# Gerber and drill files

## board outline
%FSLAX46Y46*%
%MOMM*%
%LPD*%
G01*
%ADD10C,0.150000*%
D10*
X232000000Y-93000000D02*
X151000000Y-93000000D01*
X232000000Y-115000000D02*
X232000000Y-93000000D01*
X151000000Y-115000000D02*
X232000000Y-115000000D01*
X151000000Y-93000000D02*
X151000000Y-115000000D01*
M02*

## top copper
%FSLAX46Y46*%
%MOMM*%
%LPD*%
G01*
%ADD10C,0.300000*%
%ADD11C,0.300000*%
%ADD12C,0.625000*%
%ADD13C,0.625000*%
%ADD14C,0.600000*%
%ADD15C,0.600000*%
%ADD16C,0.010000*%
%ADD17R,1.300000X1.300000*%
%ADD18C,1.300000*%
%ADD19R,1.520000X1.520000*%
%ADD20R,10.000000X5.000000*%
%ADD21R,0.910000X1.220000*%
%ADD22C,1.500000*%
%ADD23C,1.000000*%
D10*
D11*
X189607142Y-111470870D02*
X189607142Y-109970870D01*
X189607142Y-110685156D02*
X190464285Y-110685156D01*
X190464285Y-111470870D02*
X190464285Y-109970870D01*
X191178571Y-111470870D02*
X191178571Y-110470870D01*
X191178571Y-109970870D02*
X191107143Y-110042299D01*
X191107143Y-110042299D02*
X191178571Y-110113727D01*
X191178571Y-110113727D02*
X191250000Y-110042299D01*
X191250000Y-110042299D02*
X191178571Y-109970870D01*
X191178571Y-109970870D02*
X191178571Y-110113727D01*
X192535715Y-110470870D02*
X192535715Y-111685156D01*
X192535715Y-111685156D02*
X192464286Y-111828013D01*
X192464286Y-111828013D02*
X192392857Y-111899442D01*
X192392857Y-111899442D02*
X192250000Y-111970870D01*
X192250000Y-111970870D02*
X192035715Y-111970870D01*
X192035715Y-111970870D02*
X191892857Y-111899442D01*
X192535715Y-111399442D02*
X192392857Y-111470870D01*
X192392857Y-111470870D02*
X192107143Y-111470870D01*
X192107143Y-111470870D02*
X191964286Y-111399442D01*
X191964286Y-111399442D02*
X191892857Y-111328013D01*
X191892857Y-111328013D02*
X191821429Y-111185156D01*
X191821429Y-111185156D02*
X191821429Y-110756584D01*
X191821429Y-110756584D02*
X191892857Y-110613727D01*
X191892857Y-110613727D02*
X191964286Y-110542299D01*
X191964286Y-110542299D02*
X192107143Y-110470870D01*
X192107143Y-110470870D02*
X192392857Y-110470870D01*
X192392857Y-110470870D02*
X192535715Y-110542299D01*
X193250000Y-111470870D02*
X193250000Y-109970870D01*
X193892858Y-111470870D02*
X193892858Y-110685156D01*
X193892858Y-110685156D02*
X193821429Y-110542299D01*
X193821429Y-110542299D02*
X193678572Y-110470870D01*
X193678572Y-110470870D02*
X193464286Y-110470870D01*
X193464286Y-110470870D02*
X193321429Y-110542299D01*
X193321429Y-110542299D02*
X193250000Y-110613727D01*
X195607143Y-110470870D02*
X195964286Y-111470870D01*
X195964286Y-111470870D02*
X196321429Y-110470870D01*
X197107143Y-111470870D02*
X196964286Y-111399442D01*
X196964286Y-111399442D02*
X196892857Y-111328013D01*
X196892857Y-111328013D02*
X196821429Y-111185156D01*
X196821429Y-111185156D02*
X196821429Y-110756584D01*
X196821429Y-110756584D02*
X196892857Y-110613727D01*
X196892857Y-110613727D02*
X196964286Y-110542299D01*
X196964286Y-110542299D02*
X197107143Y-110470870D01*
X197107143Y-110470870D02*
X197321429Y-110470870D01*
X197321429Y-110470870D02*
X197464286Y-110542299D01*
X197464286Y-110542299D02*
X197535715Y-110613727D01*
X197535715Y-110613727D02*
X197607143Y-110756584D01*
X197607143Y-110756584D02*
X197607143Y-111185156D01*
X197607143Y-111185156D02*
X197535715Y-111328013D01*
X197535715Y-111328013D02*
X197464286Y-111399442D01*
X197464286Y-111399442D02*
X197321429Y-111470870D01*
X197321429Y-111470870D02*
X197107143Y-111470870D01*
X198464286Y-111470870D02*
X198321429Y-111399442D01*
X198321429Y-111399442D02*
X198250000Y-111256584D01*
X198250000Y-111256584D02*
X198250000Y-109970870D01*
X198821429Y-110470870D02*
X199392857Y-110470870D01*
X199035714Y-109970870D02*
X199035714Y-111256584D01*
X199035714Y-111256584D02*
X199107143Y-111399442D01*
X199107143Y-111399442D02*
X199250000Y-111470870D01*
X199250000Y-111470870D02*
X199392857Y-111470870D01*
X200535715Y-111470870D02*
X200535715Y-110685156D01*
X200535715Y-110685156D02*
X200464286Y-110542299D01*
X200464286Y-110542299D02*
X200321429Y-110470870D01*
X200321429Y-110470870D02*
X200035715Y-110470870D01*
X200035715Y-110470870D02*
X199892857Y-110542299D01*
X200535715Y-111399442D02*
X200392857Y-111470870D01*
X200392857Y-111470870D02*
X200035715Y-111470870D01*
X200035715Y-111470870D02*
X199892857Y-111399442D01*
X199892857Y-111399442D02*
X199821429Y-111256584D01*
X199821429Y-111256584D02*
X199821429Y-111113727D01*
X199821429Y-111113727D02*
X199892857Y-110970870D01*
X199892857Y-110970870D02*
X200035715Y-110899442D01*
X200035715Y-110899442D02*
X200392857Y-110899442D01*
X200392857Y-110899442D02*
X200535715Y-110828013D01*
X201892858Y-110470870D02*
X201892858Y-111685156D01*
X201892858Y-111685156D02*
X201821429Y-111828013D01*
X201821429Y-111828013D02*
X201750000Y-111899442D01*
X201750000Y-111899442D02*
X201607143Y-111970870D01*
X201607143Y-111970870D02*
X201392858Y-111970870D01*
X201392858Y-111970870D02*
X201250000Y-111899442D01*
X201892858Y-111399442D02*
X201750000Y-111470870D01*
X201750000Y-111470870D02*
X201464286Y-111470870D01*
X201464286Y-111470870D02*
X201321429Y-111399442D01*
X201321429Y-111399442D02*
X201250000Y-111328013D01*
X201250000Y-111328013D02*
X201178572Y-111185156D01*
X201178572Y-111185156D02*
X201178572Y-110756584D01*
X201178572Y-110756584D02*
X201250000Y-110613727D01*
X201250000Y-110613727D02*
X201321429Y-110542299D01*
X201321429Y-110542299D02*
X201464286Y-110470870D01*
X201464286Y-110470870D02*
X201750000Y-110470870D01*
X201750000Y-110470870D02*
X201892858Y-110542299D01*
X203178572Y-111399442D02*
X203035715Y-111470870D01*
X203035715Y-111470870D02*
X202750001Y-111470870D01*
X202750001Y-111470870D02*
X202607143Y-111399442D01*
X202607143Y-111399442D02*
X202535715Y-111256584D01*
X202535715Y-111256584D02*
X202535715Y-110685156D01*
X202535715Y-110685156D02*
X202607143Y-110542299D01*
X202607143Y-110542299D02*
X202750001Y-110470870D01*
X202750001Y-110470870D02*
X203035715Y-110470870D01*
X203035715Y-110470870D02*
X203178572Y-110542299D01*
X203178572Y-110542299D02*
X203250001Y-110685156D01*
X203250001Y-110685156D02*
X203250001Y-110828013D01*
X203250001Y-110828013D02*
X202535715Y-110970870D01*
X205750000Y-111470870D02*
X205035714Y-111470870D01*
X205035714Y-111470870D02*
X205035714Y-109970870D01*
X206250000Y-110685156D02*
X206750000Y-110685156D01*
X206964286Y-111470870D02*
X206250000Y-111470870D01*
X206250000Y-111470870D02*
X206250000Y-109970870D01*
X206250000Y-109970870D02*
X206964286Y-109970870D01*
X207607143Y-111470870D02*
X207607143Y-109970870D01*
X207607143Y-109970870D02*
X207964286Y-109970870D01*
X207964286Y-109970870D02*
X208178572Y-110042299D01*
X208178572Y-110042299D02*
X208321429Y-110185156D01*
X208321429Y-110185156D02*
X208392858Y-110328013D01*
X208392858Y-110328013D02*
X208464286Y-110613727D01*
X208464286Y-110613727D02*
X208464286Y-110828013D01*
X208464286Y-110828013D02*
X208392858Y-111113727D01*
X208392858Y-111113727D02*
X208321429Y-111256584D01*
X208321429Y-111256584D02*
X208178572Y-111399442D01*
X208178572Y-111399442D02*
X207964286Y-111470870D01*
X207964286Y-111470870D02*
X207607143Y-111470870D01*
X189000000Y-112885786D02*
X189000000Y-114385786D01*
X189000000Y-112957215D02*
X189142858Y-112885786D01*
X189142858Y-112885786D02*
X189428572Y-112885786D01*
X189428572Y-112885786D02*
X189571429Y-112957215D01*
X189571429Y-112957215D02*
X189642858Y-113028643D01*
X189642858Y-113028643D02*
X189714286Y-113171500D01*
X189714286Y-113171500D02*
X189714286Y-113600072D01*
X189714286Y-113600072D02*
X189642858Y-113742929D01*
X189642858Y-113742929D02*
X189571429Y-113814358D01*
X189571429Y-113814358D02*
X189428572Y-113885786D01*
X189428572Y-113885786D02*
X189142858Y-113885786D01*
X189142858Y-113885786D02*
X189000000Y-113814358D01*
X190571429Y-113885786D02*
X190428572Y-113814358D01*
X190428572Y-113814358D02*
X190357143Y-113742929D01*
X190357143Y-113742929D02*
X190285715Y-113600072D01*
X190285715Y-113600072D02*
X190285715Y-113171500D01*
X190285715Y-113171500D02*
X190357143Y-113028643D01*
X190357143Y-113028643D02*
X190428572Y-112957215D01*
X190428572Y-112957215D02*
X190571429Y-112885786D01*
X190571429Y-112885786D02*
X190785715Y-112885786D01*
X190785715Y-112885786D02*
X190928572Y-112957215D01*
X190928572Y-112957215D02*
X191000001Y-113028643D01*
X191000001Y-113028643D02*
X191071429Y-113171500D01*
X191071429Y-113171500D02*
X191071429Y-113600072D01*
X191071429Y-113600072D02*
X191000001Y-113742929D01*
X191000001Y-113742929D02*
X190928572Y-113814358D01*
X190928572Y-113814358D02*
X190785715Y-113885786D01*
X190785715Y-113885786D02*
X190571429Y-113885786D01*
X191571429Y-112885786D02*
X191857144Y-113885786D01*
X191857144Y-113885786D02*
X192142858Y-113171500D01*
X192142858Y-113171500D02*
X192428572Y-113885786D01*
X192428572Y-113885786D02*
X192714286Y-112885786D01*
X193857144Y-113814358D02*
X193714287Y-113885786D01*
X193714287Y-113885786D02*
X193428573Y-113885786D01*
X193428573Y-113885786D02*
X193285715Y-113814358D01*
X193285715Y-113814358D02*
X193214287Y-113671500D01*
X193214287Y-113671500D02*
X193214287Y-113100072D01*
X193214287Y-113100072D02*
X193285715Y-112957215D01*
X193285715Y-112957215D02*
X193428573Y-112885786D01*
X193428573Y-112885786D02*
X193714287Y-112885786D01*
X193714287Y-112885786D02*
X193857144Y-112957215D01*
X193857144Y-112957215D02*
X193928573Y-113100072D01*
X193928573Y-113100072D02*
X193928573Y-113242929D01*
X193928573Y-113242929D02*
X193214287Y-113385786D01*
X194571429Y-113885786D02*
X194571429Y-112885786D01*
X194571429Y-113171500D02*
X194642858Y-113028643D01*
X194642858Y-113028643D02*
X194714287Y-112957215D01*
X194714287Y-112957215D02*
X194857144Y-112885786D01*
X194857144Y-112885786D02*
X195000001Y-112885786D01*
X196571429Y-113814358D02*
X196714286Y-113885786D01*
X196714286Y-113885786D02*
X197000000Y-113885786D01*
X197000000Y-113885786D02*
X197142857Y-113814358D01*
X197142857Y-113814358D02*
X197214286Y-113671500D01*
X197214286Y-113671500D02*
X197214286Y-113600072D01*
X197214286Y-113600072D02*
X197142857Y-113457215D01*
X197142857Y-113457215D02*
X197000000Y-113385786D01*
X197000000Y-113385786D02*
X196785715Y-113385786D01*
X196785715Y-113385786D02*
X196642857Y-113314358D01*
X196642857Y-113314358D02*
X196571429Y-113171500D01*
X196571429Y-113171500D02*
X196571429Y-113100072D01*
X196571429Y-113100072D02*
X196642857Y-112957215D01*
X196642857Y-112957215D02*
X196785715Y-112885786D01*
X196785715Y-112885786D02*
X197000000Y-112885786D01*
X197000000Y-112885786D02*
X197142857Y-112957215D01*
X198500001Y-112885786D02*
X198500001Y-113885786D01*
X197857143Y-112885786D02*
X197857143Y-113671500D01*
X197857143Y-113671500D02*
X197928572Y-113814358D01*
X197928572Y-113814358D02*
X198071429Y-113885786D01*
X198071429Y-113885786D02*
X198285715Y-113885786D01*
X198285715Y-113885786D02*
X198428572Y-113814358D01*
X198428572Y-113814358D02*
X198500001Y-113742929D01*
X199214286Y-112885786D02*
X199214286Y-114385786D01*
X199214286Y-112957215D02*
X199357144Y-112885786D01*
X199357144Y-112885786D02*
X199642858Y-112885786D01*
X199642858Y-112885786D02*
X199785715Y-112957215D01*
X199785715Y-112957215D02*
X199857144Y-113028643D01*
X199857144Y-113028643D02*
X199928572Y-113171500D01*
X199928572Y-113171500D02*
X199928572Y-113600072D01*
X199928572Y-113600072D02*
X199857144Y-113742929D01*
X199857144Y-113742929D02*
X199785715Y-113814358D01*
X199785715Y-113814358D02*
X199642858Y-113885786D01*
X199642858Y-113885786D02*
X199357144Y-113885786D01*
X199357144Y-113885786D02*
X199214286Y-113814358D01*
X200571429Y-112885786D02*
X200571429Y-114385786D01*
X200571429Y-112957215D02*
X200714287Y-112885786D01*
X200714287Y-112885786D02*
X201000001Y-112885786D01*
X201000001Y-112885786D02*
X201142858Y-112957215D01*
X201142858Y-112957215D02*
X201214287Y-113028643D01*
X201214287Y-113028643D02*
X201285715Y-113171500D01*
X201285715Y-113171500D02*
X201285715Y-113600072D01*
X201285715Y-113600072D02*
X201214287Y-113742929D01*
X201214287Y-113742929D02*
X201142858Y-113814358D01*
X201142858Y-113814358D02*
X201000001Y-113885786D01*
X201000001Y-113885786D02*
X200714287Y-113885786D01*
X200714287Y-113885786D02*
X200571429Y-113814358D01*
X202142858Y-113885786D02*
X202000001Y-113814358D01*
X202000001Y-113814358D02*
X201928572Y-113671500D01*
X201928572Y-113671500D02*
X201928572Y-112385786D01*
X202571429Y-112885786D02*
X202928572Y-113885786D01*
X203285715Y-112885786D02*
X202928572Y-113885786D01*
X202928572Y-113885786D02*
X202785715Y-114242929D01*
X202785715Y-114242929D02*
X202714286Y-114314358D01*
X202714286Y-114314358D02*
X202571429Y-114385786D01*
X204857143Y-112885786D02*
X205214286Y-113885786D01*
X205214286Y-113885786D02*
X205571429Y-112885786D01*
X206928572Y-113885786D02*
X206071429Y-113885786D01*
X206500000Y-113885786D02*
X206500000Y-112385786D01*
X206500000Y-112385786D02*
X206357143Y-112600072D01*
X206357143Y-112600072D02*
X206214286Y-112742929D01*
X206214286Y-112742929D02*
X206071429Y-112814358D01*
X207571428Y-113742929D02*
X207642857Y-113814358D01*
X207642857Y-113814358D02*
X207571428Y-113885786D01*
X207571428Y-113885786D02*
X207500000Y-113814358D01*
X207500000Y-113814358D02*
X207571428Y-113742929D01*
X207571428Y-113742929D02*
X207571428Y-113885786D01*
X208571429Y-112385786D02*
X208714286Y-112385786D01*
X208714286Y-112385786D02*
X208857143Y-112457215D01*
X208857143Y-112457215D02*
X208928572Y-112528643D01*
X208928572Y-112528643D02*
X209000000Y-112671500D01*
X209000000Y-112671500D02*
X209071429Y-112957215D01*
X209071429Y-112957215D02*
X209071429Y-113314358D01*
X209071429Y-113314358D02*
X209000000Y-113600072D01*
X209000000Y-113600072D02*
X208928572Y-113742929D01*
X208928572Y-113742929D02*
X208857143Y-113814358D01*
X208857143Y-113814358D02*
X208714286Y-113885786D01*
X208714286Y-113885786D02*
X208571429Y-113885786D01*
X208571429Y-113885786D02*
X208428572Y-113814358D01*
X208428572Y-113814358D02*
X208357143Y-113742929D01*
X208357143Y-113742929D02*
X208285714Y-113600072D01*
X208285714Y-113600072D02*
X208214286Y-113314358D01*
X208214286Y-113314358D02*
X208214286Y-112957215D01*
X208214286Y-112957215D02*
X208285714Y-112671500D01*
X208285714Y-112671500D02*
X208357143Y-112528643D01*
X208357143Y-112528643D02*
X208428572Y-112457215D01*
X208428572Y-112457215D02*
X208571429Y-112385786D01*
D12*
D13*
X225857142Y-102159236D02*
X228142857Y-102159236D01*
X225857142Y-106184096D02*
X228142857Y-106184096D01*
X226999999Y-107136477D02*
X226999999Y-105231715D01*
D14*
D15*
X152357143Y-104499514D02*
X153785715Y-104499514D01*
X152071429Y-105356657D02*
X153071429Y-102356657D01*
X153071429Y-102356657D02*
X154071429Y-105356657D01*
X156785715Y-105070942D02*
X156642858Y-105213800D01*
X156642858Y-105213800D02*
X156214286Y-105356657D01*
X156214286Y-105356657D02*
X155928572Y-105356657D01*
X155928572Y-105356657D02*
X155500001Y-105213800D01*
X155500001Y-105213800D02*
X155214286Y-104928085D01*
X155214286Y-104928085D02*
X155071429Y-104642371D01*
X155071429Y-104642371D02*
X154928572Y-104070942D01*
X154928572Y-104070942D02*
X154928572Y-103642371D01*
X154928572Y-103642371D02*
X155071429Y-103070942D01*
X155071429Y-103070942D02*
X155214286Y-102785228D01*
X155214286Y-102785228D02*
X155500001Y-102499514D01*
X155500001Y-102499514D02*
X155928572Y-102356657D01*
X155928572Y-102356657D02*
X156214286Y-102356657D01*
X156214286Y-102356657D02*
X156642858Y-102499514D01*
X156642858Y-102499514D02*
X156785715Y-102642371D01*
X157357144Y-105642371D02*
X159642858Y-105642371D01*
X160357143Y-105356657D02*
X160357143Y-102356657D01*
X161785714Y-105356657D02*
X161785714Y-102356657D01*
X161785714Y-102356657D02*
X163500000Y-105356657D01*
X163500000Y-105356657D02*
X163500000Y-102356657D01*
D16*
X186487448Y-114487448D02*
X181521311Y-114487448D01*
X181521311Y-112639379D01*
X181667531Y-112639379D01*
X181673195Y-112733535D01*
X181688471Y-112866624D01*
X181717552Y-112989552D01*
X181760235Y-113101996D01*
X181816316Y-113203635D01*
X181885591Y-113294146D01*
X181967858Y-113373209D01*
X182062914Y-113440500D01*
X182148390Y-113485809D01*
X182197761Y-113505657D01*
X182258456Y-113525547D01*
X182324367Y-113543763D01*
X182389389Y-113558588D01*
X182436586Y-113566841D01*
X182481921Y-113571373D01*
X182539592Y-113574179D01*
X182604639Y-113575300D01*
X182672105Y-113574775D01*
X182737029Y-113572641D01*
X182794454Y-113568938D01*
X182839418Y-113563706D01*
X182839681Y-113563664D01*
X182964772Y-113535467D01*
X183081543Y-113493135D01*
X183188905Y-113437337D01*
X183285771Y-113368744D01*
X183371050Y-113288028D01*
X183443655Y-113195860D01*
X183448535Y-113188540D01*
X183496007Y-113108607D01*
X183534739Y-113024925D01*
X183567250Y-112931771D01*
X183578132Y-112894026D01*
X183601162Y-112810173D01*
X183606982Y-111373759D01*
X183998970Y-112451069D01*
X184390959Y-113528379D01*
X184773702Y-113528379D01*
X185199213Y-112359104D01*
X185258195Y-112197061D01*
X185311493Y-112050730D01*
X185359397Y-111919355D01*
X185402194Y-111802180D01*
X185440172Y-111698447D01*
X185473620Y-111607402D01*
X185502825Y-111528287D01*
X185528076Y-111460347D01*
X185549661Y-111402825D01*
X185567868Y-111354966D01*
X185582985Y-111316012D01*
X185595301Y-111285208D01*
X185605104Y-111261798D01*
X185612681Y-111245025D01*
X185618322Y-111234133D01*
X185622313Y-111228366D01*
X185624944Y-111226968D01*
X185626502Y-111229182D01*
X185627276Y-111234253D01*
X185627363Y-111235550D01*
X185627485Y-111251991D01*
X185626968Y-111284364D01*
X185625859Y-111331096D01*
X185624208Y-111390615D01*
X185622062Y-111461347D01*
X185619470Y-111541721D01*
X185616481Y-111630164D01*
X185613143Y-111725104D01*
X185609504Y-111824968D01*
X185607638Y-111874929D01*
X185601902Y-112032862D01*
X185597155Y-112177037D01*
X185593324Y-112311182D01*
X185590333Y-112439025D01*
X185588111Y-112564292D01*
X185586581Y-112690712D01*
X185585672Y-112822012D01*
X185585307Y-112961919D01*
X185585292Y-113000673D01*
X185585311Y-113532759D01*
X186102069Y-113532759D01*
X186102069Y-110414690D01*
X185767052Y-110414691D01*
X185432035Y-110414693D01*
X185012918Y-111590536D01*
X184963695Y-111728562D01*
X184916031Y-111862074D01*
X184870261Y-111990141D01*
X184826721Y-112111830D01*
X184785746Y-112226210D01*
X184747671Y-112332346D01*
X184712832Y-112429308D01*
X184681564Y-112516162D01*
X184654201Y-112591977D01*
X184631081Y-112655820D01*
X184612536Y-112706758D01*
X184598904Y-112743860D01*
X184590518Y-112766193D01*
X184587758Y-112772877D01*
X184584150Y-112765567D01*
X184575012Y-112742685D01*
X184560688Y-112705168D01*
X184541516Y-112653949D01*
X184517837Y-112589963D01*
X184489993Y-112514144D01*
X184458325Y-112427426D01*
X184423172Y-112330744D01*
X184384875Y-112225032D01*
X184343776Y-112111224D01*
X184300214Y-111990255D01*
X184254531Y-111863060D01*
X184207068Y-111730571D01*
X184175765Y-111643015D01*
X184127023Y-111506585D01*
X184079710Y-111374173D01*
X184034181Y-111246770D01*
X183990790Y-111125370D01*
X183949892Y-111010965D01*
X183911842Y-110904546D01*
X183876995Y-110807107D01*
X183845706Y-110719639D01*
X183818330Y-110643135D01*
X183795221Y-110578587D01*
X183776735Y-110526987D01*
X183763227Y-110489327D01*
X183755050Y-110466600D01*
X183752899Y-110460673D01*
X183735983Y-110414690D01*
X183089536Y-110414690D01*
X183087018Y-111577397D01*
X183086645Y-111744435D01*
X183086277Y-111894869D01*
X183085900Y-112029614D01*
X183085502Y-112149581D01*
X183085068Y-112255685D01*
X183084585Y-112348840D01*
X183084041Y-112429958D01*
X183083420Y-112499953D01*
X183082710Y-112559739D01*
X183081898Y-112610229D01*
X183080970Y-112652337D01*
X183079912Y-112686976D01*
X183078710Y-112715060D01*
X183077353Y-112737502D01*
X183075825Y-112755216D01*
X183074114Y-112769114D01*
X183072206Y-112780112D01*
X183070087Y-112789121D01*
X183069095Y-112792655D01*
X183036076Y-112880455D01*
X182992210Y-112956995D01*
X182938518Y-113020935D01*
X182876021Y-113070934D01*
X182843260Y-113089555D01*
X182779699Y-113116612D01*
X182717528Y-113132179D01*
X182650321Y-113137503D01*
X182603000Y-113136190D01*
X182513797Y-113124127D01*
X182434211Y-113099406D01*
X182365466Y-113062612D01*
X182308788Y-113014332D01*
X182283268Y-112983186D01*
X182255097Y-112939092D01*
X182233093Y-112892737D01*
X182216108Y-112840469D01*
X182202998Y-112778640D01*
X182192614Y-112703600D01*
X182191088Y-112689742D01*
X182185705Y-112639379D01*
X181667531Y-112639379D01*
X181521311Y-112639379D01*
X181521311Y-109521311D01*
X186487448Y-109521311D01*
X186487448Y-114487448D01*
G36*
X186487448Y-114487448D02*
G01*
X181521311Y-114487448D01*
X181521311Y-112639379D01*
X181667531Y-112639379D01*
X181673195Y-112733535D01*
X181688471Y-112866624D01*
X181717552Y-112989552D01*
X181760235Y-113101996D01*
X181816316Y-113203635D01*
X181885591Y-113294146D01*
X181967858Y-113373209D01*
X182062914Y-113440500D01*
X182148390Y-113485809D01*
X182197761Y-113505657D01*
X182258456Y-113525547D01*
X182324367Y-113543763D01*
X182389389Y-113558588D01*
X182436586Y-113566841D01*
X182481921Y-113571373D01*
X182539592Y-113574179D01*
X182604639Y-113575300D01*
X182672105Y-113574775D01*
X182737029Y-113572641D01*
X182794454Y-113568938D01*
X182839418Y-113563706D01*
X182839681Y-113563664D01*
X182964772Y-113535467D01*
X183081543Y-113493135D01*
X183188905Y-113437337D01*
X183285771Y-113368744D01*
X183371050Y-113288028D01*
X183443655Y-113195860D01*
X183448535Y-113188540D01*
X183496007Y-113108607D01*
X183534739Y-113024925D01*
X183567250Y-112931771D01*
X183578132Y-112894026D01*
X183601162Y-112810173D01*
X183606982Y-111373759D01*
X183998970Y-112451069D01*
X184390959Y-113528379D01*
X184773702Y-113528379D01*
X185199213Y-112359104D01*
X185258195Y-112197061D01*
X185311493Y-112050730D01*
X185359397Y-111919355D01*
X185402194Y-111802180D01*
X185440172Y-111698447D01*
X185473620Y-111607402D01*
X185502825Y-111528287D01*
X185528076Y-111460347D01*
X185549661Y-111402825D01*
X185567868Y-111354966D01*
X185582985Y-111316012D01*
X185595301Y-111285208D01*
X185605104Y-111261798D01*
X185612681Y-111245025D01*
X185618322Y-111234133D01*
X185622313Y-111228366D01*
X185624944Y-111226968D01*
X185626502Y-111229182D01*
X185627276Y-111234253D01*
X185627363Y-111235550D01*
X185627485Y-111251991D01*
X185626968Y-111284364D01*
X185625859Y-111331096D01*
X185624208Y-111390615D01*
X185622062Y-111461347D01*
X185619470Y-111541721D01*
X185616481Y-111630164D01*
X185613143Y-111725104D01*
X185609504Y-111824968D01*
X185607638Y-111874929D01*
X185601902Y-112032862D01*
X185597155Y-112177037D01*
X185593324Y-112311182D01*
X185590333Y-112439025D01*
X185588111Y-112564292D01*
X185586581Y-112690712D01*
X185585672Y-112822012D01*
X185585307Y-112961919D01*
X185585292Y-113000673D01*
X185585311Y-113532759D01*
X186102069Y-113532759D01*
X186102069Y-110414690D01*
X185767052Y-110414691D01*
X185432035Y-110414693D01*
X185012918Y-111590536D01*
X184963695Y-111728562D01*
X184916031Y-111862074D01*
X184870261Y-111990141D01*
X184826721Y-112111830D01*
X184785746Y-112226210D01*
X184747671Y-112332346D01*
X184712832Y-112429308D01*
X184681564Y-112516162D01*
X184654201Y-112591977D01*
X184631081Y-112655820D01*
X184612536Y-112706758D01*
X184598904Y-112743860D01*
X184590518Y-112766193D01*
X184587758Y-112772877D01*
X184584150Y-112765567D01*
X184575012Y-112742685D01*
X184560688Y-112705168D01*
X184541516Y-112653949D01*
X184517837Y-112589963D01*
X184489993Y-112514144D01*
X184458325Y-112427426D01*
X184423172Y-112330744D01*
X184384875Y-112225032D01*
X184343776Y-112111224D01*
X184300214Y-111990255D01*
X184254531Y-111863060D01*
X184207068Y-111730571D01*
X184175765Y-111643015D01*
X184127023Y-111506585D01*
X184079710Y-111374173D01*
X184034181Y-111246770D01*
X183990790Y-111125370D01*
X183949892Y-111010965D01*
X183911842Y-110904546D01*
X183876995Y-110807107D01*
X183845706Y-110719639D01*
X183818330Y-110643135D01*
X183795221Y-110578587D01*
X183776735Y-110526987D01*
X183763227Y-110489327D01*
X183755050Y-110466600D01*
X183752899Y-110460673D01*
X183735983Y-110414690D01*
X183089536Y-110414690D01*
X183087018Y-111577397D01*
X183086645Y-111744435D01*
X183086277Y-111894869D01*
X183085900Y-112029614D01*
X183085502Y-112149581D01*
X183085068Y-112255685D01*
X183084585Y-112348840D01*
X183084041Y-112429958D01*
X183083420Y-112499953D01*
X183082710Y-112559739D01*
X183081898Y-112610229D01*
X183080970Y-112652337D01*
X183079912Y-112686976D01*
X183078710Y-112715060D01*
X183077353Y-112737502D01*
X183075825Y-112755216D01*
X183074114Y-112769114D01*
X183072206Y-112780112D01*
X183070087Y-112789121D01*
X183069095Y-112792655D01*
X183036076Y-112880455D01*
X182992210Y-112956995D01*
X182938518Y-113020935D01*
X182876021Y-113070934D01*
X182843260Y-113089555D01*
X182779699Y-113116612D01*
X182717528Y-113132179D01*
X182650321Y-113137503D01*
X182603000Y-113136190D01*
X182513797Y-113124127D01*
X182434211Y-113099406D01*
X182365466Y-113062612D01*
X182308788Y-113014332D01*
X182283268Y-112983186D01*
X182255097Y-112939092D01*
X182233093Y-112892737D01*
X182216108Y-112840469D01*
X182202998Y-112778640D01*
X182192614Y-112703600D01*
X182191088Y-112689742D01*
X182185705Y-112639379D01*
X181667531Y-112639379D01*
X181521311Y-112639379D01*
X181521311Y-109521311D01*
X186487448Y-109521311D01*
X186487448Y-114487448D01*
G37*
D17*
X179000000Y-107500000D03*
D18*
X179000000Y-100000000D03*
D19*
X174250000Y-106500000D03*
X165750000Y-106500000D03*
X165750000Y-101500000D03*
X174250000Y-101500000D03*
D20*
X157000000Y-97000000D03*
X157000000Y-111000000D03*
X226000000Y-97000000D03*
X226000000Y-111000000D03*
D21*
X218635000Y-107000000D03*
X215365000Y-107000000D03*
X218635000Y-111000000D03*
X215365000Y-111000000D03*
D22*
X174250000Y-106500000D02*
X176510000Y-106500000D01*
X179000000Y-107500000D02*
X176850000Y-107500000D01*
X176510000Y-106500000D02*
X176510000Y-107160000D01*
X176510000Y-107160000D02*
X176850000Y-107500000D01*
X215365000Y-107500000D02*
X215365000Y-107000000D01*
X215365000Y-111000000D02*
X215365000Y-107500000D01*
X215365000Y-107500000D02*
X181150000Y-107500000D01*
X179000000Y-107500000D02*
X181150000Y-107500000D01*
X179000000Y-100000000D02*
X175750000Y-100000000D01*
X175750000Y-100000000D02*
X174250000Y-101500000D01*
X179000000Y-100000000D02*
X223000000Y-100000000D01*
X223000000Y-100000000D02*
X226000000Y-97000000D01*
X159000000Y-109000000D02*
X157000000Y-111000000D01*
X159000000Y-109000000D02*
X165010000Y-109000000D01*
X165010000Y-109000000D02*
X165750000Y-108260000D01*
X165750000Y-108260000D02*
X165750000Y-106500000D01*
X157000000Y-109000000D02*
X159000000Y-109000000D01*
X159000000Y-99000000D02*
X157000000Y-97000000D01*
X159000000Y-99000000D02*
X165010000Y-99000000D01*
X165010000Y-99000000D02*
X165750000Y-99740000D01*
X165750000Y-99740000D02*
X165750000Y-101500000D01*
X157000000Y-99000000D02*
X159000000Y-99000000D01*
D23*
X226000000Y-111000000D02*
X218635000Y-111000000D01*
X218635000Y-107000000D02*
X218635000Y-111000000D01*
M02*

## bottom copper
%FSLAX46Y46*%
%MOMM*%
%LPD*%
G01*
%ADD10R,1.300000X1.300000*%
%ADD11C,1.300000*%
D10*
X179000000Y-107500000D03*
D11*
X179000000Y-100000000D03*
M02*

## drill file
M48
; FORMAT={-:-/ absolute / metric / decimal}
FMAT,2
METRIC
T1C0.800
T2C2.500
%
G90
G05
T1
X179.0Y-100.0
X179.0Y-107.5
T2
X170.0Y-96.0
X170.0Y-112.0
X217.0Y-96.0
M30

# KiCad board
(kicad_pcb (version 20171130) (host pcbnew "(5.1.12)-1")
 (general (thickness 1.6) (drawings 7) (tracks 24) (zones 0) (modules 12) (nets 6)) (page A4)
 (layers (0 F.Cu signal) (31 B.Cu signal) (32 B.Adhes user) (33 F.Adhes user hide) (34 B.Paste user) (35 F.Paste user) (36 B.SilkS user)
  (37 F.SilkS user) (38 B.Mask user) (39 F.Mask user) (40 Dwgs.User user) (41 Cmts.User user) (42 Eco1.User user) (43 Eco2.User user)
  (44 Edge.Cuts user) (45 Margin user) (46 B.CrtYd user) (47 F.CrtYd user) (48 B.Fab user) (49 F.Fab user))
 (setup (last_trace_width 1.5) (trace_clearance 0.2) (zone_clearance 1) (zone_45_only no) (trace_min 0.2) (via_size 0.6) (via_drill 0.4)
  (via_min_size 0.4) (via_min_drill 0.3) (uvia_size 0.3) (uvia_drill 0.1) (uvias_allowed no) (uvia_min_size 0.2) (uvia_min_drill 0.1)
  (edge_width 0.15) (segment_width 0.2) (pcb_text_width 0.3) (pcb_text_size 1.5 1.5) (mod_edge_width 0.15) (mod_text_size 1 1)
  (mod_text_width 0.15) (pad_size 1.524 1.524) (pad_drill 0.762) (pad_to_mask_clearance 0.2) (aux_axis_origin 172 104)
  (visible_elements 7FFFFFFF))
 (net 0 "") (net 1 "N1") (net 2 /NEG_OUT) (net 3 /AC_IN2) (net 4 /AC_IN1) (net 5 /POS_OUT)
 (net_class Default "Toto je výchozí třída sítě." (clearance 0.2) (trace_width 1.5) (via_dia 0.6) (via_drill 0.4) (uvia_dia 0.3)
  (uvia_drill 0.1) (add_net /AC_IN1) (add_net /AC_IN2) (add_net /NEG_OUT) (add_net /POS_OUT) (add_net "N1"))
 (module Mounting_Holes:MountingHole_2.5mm (layer F.Cu) (at 217 96)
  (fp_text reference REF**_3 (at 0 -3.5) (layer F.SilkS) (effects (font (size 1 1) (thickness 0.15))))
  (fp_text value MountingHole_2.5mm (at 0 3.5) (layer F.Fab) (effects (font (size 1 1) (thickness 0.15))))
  (pad 1 np_thru_hole circle (at 0 0) (size 2.5 2.5) (drill 2.5) (layers *.Cu *.Mask F.SilkS)))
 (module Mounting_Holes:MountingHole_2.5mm (layer F.Cu) (at 170 96)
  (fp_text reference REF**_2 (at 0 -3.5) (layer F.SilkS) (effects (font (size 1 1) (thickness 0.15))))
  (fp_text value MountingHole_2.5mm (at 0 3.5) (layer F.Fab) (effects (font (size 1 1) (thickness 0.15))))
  (pad 1 np_thru_hole circle (at 0 0) (size 2.5 2.5) (drill 2.5) (layers *.Cu *.Mask F.SilkS)))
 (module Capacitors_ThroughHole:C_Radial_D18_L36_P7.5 (layer F.Cu) (at 179 107.5 90)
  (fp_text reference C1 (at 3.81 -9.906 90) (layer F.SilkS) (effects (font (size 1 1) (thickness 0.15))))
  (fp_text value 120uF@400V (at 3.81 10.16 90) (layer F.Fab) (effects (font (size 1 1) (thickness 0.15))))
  (pad 1 thru_hole rect (at 0 0 90) (size 1.3 1.3) (drill 0.8) (layers *.Cu *.Mask F.SilkS) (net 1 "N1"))
  (pad 2 thru_hole circle (at 7.5 0 90) (size 1.3 1.3) (drill 0.8) (layers *.Cu *.Mask F.SilkS) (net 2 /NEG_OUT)))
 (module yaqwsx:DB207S (layer F.Cu) (at 170 104 270)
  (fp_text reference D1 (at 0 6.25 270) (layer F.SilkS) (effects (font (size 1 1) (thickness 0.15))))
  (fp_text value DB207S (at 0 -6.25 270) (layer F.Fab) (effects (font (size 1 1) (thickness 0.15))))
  (pad 3 smd rect (at 2.5 -4.25 270) (size 1.52 1.52) (layers F.Cu F.Paste F.Mask) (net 1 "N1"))
  (pad 4 smd rect (at 2.5 4.25 270) (size 1.52 1.52) (layers F.Cu F.Paste F.Mask) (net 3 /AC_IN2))
  (pad 2 smd rect (at -2.5 4.25 270) (size 1.52 1.52) (layers F.Cu F.Paste F.Mask) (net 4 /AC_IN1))
  (pad 1 smd rect (at -2.5 -4.25 270) (size 1.52 1.52) (layers F.Cu F.Paste F.Mask) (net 2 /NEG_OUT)))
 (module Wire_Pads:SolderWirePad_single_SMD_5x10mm (layer F.Cu) (at 157 97 90)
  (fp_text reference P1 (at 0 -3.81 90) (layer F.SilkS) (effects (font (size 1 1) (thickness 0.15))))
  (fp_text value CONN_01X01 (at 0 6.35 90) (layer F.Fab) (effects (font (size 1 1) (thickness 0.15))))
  (pad 1 smd rect (at 0 0 90) (size 5 10) (layers F.Cu F.Paste F.Mask) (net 4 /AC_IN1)))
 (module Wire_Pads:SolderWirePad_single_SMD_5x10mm (layer F.Cu) (at 157 111 90)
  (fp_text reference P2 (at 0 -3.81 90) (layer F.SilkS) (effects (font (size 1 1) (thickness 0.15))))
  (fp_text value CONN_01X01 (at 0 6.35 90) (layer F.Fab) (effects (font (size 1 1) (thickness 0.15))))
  (pad 1 smd rect (at 0 0 90) (size 5 10) (layers F.Cu F.Paste F.Mask) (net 3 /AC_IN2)))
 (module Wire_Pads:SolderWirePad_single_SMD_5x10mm (layer F.Cu) (at 226 97 90)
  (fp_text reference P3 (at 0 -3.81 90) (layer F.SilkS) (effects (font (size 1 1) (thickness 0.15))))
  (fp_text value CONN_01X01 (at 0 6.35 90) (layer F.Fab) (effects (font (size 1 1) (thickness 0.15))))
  (pad 1 smd rect (at 0 0 90) (size 5 10) (layers F.Cu F.Paste F.Mask) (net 2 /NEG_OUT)))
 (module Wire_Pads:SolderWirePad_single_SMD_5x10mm (layer F.Cu) (at 226 111 90)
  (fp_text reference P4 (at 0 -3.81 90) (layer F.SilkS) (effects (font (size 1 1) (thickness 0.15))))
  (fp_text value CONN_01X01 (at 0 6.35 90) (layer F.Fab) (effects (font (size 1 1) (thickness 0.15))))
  (pad 1 smd rect (at 0 0 90) (size 5 10) (layers F.Cu F.Paste F.Mask) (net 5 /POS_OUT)))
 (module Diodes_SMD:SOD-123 (layer F.Cu) (at 217 107 180)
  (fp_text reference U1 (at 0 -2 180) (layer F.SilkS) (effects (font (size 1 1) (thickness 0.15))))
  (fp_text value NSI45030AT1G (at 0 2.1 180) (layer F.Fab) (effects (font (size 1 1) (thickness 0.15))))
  (pad 1 smd rect (at -1.635 0 180) (size 0.91 1.22) (layers F.Cu F.Paste F.Mask) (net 5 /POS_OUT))
  (pad 2 smd rect (at 1.635 0 180) (size 0.91 1.22) (layers F.Cu F.Paste F.Mask) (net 1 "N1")))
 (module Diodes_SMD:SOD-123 (layer F.Cu) (at 217 111 180)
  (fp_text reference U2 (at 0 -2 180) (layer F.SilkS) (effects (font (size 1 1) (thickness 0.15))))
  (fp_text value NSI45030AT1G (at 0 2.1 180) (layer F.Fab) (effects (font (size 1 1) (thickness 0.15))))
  (pad 1 smd rect (at -1.635 0 180) (size 0.91 1.22) (layers F.Cu F.Paste F.Mask) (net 5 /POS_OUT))
  (pad 2 smd rect (at 1.635 0 180) (size 0.91 1.22) (layers F.Cu F.Paste F.Mask) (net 1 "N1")))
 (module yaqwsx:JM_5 (layer F.Cu) (at 184 112)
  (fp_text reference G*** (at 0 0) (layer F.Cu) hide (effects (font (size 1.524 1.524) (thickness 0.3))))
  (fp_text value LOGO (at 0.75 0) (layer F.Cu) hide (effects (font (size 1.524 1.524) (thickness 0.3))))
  (fp_poly
   (pts (xy 2.487448 2.487448) (xy -2.478689 2.487448) (xy -2.478689 0.639379) (xy -2.332469 0.639379) (xy -2.326805 0.733535)
    (xy -2.311529 0.866624) (xy -2.282448 0.989552) (xy -2.239765 1.101996) (xy -2.183684 1.203635) (xy -2.114409 1.294146)
    (xy -2.032142 1.373209) (xy -1.937086 1.4405) (xy -1.85161 1.485809) (xy -1.802239 1.505657) (xy -1.741544 1.525547)
    (xy -1.675633 1.543763) (xy -1.610611 1.558588) (xy -1.563414 1.566841) (xy -1.518079 1.571373) (xy -1.460408 1.574179)
    (xy -1.395361 1.5753) (xy -1.327895 1.574775) (xy -1.262971 1.572641) (xy -1.205546 1.568938) (xy -1.160582 1.563706)
    (xy -1.160319 1.563664) (xy -1.035228 1.535467) (xy -0.918457 1.493135) (xy -0.811095 1.437337) (xy -0.714229 1.368744)
    (xy -0.62895 1.288028) (xy -0.556345 1.19586) (xy -0.551465 1.18854) (xy -0.503993 1.108607) (xy -0.465261 1.024925)
    (xy -0.43275 0.931771) (xy -0.421868 0.894026) (xy -0.398838 0.810173) (xy -0.393018 -0.626241) (xy -0.00103 0.451069)
    (xy 0.390959 1.528379) (xy 0.773702 1.528379) (xy 1.199213 0.359104) (xy 1.258195 0.197061) (xy 1.311493 0.05073)
    (xy 1.359397 -0.080645) (xy 1.402194 -0.19782) (xy 1.440172 -0.301553) (xy 1.47362 -0.392598) (xy 1.502825 -0.471713)
    (xy 1.528076 -0.539653) (xy 1.549661 -0.597175) (xy 1.567868 -0.645034) (xy 1.582985 -0.683988) (xy 1.595301 -0.714792)
    (xy 1.605104 -0.738202) (xy 1.612681 -0.754975) (xy 1.618322 -0.765867) (xy 1.622313 -0.771634) (xy 1.624944 -0.773032)
    (xy 1.626502 -0.770818) (xy 1.627276 -0.765747) (xy 1.627363 -0.76445) (xy 1.627485 -0.748009) (xy 1.626968 -0.715636)
    (xy 1.625859 -0.668904) (xy 1.624208 -0.609385) (xy 1.622062 -0.538653) (xy 1.61947 -0.458279) (xy 1.616481 -0.369836)
    (xy 1.613143 -0.274896) (xy 1.609504 -0.175032) (xy 1.607638 -0.125071) (xy 1.601902 0.032862) (xy 1.597155 0.177037)
    (xy 1.593324 0.311182) (xy 1.590333 0.439025) (xy 1.588111 0.564292) (xy 1.586581 0.690712) (xy 1.585672 0.822012)
    (xy 1.585307 0.961919) (xy 1.585292 1.000673) (xy 1.585311 1.532759) (xy 2.102069 1.532759) (xy 2.102069 -1.58531)
    (xy 1.767052 -1.585309) (xy 1.432035 -1.585307) (xy 1.012918 -0.409464) (xy 0.963695 -0.271438) (xy 0.916031 -0.137926)
    (xy 0.870261 -0.009859) (xy 0.826721 0.11183) (xy 0.785746 0.22621) (xy 0.747671 0.332346) (xy 0.712832 0.429308) (xy 0.681564 0.516162)
    (xy 0.654201 0.591977) (xy 0.631081 0.65582) (xy 0.612536 0.706758) (xy 0.598904 0.74386) (xy 0.590518 0.766193) (xy 0.587758 0.772877)
    (xy 0.58415 0.765567) (xy 0.575012 0.742685) (xy 0.560688 0.705168) (xy 0.541516 0.653949) (xy 0.517837 0.589963) (xy 0.489993 0.514144)
    (xy 0.458325 0.427426) (xy 0.423172 0.330744) (xy 0.384875 0.225032) (xy 0.343776 0.111224) (xy 0.300214 -0.009745)
    (xy 0.254531 -0.13694) (xy 0.207068 -0.269429) (xy 0.175765 -0.356985) (xy 0.127023 -0.493415) (xy 0.07971 -0.625827)
    (xy 0.034181 -0.75323) (xy -0.00921 -0.87463) (xy -0.050108 -0.989035) (xy -0.088158 -1.095454) (xy -0.123005 -1.192893)
    (xy -0.154294 -1.280361) (xy -0.18167 -1.356865) (xy -0.204779 -1.421413) (xy -0.223265 -1.473013) (xy -0.236773 -1.510673)
    (xy -0.24495 -1.5334) (xy -0.247101 -1.539327) (xy -0.264017 -1.58531) (xy -0.910464 -1.58531) (xy -0.912982 -0.422603)
    (xy -0.913355 -0.255565) (xy -0.913723 -0.105131) (xy -0.9141 0.029614) (xy -0.914498 0.149581) (xy -0.914932 0.255685)
    (xy -0.915415 0.34884) (xy -0.915959 0.429958) (xy -0.91658 0.499953) (xy -0.91729 0.559739) (xy -0.918102 0.610229)
    (xy -0.91903 0.652337) (xy -0.920088 0.686976) (xy -0.92129 0.71506) (xy -0.922647 0.737502) (xy -0.924175 0.755216)
    (xy -0.925886 0.769114) (xy -0.927794 0.780112) (xy -0.929913 0.789121) (xy -0.930905 0.792655) (xy -0.963924 0.880455)
    (xy -1.00779 0.956995) (xy -1.061482 1.020935) (xy -1.123979 1.070934) (xy -1.15674 1.089555) (xy -1.220301 1.116612)
    (xy -1.282472 1.132179) (xy -1.349679 1.137503) (xy -1.397 1.13619) (xy -1.486203 1.124127) (xy -1.565789 1.099406)
    (xy -1.634534 1.062612) (xy -1.691212 1.014332) (xy -1.716732 0.983186) (xy -1.744903 0.939092) (xy -1.766907 0.892737)
    (xy -1.783892 0.840469) (xy -1.797002 0.77864) (xy -1.807386 0.7036) (xy -1.808912 0.689742) (xy -1.814295 0.639379)
    (xy -2.332469 0.639379) (xy -2.478689 0.639379) (xy -2.478689 -2.478689) (xy 2.487448 -2.478689) (xy 2.487448 2.487448))
   (layer F.Cu) (width 0.01)))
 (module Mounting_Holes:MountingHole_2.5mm (layer F.Cu) (at 170 112)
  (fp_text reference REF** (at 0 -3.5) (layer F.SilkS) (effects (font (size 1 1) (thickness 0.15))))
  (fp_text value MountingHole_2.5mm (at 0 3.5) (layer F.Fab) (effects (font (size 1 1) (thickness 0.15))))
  (pad 1 np_thru_hole circle (at 0 0) (size 2.5 2.5) (drill 2.5) (layers *.Cu *.Mask F.SilkS)))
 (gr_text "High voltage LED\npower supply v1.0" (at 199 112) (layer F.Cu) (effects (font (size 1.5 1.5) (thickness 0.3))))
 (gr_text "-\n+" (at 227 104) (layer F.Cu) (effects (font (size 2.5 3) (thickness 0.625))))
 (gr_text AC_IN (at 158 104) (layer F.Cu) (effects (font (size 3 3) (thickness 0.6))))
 (gr_line (start 232 93) (end 151 93) (layer Edge.Cuts) (width 0.15))
 (gr_line (start 232 115) (end 232 93) (layer Edge.Cuts) (width 0.15))
 (gr_line (start 151 115) (end 232 115) (layer Edge.Cuts) (width 0.15))
 (gr_line (start 151 93) (end 151 115) (layer Edge.Cuts) (width 0.15))
 (segment (start 174.25 106.5) (end 176.51 106.5) (width 1.5) (layer F.Cu) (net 1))
 (segment (start 179 107.5) (end 176.85 107.5) (width 1.5) (layer F.Cu) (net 1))
 (segment (start 176.51 106.5) (end 176.51 107.16) (width 1.5) (layer F.Cu) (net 1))
 (segment (start 176.51 107.16) (end 176.85 107.5) (width 1.5) (layer F.Cu) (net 1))
 (segment (start 215.365 107.5) (end 215.365 107) (width 1.5) (layer F.Cu) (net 1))
 (segment (start 215.365 111) (end 215.365 107.5) (width 1.5) (layer F.Cu) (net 1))
 (segment (start 215.365 107.5) (end 181.15 107.5) (width 1.5) (layer F.Cu) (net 1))
 (segment (start 179 107.5) (end 181.15 107.5) (width 1.5) (layer F.Cu) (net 1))
 (segment (start 179 100) (end 175.75 100) (width 1.5) (layer F.Cu) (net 2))
 (segment (start 175.75 100) (end 174.25 101.5) (width 1.5) (layer F.Cu) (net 2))
 (segment (start 179 100) (end 223 100) (width 1.5) (layer F.Cu) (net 2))
 (segment (start 223 100) (end 226 97) (width 1.5) (layer F.Cu) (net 2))
 (segment (start 159 109) (end 157 111) (width 1.5) (layer F.Cu) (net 3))
 (segment (start 159 109) (end 165.01 109) (width 1.5) (layer F.Cu) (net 3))
 (segment (start 165.01 109) (end 165.75 108.26) (width 1.5) (layer F.Cu) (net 3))
 (segment (start 165.75 108.26) (end 165.75 106.5) (width 1.5) (layer F.Cu) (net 3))
 (segment (start 157 109) (end 159 109) (width 1.5) (layer F.Cu) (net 3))
 (segment (start 159 99) (end 157 97) (width 1.5) (layer F.Cu) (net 4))
 (segment (start 159 99) (end 165.01 99) (width 1.5) (layer F.Cu) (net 4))
 (segment (start 165.01 99) (end 165.75 99.74) (width 1.5) (layer F.Cu) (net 4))
 (segment (start 165.75 99.74) (end 165.75 101.5) (width 1.5) (layer F.Cu) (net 4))
 (segment (start 157 99) (end 159 99) (width 1.5) (layer F.Cu) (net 4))
 (segment (start 226 111) (end 218.635 111) (width 1) (layer F.Cu) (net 5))
 (segment (start 218.635 107) (end 218.635 111) (width 1) (layer F.Cu) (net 5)))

